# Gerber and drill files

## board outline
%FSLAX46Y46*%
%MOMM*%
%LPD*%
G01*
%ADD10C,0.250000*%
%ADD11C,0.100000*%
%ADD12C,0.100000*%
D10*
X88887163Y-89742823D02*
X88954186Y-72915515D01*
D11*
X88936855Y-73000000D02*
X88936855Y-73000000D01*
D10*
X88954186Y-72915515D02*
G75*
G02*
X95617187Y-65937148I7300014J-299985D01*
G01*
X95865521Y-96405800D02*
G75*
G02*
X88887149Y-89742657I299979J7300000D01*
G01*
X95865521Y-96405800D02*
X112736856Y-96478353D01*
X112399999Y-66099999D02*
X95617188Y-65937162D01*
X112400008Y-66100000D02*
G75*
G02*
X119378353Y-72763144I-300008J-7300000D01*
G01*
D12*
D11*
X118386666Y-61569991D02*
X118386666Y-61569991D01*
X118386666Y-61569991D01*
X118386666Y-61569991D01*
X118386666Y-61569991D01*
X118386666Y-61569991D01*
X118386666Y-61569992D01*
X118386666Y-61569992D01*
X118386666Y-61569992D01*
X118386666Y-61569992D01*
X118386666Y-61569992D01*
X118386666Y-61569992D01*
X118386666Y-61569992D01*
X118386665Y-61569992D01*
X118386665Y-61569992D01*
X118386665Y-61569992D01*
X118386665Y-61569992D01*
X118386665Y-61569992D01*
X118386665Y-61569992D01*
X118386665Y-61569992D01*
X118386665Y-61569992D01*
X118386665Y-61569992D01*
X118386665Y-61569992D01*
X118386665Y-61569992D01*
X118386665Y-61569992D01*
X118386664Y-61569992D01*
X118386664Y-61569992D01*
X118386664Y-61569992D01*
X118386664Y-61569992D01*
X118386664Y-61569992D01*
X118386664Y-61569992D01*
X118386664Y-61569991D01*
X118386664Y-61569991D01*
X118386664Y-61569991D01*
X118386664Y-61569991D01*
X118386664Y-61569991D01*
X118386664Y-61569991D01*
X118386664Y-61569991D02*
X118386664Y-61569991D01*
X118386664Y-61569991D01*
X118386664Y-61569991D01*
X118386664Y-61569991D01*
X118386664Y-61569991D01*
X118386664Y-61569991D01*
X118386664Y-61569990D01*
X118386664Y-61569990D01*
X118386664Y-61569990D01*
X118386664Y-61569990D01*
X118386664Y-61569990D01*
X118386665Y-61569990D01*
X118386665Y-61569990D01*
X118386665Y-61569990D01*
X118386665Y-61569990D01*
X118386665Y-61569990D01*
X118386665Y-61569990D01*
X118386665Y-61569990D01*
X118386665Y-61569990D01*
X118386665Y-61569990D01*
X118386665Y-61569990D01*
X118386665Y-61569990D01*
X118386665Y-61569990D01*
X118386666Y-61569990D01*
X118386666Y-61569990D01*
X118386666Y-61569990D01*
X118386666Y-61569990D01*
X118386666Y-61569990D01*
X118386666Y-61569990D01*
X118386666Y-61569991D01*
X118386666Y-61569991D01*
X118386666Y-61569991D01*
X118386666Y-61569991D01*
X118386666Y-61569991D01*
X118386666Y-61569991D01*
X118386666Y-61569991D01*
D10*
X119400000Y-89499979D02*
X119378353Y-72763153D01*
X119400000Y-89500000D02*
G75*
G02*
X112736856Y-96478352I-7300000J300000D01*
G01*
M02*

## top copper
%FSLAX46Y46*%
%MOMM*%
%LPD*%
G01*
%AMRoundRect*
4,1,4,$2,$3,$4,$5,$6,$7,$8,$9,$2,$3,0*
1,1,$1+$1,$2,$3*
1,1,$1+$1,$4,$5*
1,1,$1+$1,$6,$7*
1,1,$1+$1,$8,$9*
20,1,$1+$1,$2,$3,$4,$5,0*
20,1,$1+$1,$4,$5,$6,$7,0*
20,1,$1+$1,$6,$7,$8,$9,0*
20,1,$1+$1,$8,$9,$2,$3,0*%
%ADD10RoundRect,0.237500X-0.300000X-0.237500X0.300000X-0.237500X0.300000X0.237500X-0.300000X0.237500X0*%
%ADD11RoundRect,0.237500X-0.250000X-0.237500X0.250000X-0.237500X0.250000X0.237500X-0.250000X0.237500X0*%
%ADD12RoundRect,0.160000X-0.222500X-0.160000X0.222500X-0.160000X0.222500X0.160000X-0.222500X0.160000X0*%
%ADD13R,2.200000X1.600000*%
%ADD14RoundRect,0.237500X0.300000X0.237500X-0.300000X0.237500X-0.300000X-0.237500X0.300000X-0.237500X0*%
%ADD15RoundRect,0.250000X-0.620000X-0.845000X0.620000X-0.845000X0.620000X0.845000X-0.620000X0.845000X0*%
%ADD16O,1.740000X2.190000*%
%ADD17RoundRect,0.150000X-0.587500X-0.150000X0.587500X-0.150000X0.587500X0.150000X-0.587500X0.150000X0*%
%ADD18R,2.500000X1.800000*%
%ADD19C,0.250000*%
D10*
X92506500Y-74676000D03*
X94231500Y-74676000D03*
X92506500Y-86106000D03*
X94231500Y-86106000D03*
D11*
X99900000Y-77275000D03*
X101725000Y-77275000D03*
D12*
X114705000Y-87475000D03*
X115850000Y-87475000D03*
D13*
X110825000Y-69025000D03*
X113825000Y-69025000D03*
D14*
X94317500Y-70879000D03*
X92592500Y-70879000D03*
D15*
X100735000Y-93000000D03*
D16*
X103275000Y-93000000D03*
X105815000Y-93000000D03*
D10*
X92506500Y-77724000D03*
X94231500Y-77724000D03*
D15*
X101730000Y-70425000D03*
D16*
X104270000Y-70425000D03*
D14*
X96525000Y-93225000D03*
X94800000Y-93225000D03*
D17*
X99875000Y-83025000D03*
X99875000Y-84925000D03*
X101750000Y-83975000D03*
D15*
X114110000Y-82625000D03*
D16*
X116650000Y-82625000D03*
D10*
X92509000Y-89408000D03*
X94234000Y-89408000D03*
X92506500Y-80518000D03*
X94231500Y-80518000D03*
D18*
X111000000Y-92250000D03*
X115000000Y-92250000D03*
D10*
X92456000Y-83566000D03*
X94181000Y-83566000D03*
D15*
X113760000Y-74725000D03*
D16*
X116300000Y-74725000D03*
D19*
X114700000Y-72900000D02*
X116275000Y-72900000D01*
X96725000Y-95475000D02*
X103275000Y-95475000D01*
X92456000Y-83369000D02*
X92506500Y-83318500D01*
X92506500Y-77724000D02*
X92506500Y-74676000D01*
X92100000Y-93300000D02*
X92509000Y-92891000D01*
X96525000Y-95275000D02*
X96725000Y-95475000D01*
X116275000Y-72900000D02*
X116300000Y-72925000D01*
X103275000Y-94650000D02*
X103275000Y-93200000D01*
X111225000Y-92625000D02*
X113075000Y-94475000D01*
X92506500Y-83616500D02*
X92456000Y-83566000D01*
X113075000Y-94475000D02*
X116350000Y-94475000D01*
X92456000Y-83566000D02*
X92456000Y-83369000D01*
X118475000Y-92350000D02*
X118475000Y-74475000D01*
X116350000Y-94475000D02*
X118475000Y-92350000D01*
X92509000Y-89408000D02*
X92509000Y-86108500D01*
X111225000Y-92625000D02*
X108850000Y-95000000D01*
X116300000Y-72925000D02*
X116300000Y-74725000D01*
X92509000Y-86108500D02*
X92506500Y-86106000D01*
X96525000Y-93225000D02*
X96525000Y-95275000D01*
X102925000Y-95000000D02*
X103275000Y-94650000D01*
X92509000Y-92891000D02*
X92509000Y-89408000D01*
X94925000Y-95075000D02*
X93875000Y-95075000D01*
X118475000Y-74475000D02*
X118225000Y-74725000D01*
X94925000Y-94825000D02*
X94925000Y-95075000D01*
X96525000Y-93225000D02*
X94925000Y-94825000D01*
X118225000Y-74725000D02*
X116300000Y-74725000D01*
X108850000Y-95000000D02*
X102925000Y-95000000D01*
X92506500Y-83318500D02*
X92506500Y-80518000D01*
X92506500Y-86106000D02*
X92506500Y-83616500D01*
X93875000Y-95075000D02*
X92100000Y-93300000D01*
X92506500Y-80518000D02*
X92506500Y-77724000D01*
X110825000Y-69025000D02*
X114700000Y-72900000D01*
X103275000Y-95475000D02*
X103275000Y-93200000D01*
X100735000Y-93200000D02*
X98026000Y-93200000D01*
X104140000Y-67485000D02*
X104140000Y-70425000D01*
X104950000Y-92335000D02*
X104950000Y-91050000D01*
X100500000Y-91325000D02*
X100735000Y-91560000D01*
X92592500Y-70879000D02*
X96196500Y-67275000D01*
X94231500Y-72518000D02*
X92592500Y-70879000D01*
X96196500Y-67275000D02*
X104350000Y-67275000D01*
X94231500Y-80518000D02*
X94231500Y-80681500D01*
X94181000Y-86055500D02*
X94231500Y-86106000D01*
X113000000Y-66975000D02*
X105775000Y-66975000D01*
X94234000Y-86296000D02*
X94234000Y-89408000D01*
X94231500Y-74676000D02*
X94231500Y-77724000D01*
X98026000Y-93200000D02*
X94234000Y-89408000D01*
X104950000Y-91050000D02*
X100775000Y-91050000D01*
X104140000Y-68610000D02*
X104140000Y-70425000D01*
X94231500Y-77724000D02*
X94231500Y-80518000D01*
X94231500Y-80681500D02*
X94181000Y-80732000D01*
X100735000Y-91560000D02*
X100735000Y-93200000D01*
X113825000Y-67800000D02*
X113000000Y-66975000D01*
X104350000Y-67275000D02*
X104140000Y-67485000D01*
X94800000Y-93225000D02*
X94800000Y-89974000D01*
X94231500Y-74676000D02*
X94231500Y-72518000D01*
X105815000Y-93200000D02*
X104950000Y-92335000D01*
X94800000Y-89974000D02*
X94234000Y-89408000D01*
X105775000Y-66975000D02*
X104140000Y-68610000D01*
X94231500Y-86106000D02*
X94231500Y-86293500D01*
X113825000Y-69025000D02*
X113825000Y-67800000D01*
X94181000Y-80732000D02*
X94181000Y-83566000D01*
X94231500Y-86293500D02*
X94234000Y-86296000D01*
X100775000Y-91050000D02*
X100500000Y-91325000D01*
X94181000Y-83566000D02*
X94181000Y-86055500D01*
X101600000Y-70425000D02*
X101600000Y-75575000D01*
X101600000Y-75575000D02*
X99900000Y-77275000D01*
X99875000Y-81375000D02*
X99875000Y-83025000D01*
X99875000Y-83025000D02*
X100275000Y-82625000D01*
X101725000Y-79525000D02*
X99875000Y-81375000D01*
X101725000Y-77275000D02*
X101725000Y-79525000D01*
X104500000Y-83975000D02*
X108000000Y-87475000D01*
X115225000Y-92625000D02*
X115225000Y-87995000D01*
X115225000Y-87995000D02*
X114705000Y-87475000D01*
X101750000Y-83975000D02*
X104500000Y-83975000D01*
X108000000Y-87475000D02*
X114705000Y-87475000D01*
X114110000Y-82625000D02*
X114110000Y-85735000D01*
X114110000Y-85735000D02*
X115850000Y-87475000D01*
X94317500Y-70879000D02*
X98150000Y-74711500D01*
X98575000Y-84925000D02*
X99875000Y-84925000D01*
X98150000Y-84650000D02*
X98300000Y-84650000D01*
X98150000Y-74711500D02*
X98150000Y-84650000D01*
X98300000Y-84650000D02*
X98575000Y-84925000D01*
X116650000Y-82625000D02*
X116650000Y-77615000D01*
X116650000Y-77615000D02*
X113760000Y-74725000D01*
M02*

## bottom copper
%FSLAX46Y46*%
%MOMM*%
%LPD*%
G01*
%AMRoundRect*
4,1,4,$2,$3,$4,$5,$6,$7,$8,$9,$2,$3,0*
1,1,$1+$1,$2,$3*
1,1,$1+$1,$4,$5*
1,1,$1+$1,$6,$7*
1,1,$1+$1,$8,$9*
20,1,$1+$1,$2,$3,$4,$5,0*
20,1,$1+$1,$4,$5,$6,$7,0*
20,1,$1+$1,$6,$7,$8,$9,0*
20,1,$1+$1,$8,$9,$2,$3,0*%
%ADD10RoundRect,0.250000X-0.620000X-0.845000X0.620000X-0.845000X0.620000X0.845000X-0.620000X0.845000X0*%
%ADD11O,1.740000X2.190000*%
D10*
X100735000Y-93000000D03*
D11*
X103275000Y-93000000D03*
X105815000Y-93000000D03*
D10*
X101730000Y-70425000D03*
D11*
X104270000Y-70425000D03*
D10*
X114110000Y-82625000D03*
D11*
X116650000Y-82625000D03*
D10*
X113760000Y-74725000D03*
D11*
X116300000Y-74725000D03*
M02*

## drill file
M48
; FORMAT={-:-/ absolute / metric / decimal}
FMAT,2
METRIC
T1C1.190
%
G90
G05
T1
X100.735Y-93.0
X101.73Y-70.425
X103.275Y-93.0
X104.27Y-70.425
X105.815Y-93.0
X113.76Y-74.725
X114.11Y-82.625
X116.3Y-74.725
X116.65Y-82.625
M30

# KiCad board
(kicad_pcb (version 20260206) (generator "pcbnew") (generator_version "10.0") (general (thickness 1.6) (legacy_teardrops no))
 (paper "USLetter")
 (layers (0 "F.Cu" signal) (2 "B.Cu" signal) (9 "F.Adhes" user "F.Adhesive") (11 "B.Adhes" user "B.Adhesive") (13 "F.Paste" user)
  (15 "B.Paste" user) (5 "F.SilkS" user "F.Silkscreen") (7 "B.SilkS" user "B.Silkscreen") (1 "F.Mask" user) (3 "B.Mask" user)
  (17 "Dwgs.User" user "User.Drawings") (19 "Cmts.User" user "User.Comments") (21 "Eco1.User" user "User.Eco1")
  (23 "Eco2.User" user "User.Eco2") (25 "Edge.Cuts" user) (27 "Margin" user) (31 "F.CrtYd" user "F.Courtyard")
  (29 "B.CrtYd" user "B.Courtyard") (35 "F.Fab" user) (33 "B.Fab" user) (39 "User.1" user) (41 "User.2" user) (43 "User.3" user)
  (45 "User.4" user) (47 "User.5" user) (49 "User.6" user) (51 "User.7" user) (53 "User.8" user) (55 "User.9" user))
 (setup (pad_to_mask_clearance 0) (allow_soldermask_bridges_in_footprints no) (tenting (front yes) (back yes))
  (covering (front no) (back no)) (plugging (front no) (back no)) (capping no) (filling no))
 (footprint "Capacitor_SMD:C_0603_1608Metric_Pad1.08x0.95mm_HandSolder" (layer "F.Cu") (at 93.369 74.676)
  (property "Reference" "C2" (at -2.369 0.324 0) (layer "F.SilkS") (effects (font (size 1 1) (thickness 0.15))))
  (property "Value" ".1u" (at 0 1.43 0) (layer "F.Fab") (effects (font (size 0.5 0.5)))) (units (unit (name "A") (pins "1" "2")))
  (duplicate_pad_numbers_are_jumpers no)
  (pad "1" smd roundrect (at -0.8625 0) (size 1.075 0.95) (layers "F.Cu" "F.Mask" "F.Paste") (roundrect_rratio 0.25) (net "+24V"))
  (pad "2" smd roundrect (at 0.8625 0) (size 1.075 0.95) (layers "F.Cu" "F.Mask" "F.Paste") (roundrect_rratio 0.25) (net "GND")))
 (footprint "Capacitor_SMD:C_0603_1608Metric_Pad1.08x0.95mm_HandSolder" (layer "F.Cu") (at 93.369 86.106)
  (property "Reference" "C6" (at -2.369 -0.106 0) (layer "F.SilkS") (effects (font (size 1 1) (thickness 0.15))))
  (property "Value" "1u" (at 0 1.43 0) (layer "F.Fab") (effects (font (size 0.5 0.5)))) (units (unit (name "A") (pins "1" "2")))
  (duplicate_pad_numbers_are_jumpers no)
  (pad "1" smd roundrect (at -0.8625 0) (size 1.075 0.95) (layers "F.Cu" "F.Mask" "F.Paste") (roundrect_rratio 0.25) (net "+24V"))
  (pad "2" smd roundrect (at 0.8625 0) (size 1.075 0.95) (layers "F.Cu" "F.Mask" "F.Paste") (roundrect_rratio 0.25) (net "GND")))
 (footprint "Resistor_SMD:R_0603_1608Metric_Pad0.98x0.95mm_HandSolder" (layer "F.Cu") (at 100.8125 77.275)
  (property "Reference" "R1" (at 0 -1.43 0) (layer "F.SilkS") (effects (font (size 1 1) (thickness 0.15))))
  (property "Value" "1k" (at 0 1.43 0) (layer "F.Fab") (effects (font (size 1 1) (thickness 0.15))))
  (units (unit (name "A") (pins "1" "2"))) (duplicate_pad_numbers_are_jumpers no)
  (pad "1" smd roundrect (at -0.9125 0) (size 0.975 0.95) (layers "F.Cu" "F.Mask" "F.Paste") (roundrect_rratio 0.25) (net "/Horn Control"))
  (pad "2" smd roundrect (at 0.9125 0) (size 0.975 0.95) (layers "F.Cu" "F.Mask" "F.Paste") (roundrect_rratio 0.25) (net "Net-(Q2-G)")))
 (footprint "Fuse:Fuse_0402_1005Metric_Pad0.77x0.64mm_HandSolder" (layer "F.Cu") (at 115.2775 87.475)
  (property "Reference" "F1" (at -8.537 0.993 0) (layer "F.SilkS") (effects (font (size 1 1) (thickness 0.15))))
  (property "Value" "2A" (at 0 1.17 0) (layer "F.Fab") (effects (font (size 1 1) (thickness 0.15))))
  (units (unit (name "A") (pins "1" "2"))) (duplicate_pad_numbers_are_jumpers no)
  (pad "1" smd roundrect (at -0.5725 0) (size 0.765 0.64) (layers "F.Cu" "F.Mask" "F.Paste") (roundrect_rratio 0.25) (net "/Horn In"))
  (pad "2" smd roundrect (at 0.5725 0) (size 0.765 0.64) (layers "F.Cu" "F.Mask" "F.Paste") (roundrect_rratio 0.25) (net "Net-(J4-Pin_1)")))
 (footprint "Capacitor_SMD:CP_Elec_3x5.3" (layer "F.Cu") (at 112.325 69.025)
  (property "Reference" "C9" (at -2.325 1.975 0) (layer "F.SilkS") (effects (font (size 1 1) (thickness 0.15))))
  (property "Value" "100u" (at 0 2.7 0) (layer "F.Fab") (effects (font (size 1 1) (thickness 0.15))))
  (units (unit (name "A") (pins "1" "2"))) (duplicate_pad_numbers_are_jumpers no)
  (pad "1" smd rect (at -1.5 0) (size 2.2 1.6) (layers "F.Cu" "F.Mask" "F.Paste") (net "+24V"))
  (pad "2" smd rect (at 1.5 0) (size 2.2 1.6) (layers "F.Cu" "F.Mask" "F.Paste") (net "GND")))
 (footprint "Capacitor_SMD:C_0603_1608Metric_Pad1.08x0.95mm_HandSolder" (layer "F.Cu") (at 93.455 70.879 180)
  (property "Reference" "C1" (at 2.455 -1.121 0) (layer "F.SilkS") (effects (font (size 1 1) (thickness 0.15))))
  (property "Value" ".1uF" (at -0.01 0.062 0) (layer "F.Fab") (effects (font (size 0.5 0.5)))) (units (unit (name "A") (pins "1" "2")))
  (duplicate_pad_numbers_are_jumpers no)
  (pad "1" smd roundrect (at -0.8625 0 180) (size 1.075 0.95) (layers "F.Cu" "F.Mask" "F.Paste") (roundrect_rratio 0.25) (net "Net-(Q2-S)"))
  (pad "2" smd roundrect (at 0.8625 0 180) (size 1.075 0.95) (layers "F.Cu" "F.Mask" "F.Paste") (roundrect_rratio 0.25) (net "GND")))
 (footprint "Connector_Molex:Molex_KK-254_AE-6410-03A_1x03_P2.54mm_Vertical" (layer "F.Cu") (at 100.735 93)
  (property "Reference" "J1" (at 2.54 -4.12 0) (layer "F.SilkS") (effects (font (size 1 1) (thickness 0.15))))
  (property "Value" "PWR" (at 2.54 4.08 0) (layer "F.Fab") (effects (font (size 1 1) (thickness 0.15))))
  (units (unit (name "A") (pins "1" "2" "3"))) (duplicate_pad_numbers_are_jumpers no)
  (pad "1" thru_hole roundrect (at 0 0) (size 1.74 2.19) (drill 1.19) (layers "*.Cu" "*.Mask") (remove_unused_layers no)
   (roundrect_rratio 0.143678) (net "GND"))
  (pad "2" thru_hole oval (at 2.54 0) (size 1.74 2.19) (drill 1.19) (layers "*.Cu" "*.Mask") (remove_unused_layers no) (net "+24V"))
  (pad "3" thru_hole oval (at 5.08 0) (size 1.74 2.19) (drill 1.19) (layers "*.Cu" "*.Mask") (remove_unused_layers no) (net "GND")))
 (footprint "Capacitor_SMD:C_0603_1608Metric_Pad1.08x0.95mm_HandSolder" (layer "F.Cu") (at 93.369 77.724)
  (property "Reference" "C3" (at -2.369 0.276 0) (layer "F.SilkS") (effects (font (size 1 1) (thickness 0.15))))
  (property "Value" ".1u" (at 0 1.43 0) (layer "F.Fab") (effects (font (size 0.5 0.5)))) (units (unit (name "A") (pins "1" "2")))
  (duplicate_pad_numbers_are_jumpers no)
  (pad "1" smd roundrect (at -0.8625 0) (size 1.075 0.95) (layers "F.Cu" "F.Mask" "F.Paste") (roundrect_rratio 0.25) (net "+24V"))
  (pad "2" smd roundrect (at 0.8625 0) (size 1.075 0.95) (layers "F.Cu" "F.Mask" "F.Paste") (roundrect_rratio 0.25) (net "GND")))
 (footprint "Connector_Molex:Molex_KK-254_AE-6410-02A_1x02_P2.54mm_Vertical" (layer "F.Cu") (at 101.73 70.425)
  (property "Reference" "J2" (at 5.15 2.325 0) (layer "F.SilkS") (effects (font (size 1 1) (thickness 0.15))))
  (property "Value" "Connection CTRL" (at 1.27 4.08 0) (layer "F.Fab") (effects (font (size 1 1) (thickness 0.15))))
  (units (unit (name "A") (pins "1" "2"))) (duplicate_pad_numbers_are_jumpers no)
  (pad "1" thru_hole roundrect (at 0 0) (size 1.74 2.19) (drill 1.19) (layers "*.Cu" "*.Mask") (remove_unused_layers no)
   (roundrect_rratio 0.143678) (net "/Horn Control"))
  (pad "2" thru_hole oval (at 2.54 0) (size 1.74 2.19) (drill 1.19) (layers "*.Cu" "*.Mask") (remove_unused_layers no) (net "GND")))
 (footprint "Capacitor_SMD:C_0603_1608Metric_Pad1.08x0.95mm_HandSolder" (layer "F.Cu") (at 95.6625 93.225 180)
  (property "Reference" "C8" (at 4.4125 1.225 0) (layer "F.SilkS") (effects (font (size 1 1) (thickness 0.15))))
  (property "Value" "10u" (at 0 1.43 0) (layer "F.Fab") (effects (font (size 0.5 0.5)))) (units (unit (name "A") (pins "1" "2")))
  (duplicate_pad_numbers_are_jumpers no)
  (pad "1" smd roundrect (at -0.8625 0 180) (size 1.075 0.95) (layers "F.Cu" "F.Mask" "F.Paste") (roundrect_rratio 0.25) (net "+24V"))
  (pad "2" smd roundrect (at 0.8625 0 180) (size 1.075 0.95) (layers "F.Cu" "F.Mask" "F.Paste") (roundrect_rratio 0.25) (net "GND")))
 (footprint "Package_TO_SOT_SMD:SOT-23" (layer "F.Cu") (at 100.8125 83.975)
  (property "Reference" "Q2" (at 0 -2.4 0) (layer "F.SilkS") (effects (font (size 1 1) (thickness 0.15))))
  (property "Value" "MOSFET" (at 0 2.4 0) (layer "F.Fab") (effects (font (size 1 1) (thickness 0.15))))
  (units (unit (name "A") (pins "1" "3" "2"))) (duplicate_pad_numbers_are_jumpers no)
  (pad "1" smd roundrect (at -0.9375 -0.95) (size 1.475 0.6) (layers "F.Cu" "F.Mask" "F.Paste") (roundrect_rratio 0.25) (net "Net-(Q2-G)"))
  (pad "2" smd roundrect (at -0.9375 0.95) (size 1.475 0.6) (layers "F.Cu" "F.Mask" "F.Paste") (roundrect_rratio 0.25) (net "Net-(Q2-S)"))
  (pad "3" smd roundrect (at 0.9375 0) (size 1.475 0.6) (layers "F.Cu" "F.Mask" "F.Paste") (roundrect_rratio 0.25) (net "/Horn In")))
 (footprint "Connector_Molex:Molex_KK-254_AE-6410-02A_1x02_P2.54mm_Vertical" (layer "F.Cu") (at 114.11 82.625)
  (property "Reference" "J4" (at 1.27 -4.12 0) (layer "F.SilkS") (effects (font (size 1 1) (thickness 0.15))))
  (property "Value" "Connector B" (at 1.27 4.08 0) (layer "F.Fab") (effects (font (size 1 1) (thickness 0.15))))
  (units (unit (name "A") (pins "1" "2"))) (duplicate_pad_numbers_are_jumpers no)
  (pad "1" thru_hole roundrect (at 0 0) (size 1.74 2.19) (drill 1.19) (layers "*.Cu" "*.Mask") (remove_unused_layers no)
   (roundrect_rratio 0.143678) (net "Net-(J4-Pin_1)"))
  (pad "2" thru_hole oval (at 2.54 0) (size 1.74 2.19) (drill 1.19) (layers "*.Cu" "*.Mask") (remove_unused_layers no)
   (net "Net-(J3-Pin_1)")))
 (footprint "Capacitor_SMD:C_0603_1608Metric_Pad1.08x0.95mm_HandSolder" (layer "F.Cu") (at 93.3715 89.408)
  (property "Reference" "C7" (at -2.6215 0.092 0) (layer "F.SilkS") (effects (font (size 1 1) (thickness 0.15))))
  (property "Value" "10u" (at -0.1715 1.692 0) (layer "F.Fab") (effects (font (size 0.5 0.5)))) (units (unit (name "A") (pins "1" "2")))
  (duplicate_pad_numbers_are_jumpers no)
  (pad "1" smd roundrect (at -0.8625 0) (size 1.075 0.95) (layers "F.Cu" "F.Mask" "F.Paste") (roundrect_rratio 0.25) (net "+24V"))
  (pad "2" smd roundrect (at 0.8625 0) (size 1.075 0.95) (layers "F.Cu" "F.Mask" "F.Paste") (roundrect_rratio 0.25) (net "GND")))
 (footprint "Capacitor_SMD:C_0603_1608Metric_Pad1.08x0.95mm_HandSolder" (layer "F.Cu") (at 93.369 80.518)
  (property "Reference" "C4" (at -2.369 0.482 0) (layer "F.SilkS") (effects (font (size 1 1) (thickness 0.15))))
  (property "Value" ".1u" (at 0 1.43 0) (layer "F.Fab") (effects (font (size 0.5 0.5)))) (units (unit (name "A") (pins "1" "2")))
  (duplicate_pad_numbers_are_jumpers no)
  (pad "1" smd roundrect (at -0.8625 0) (size 1.075 0.95) (layers "F.Cu" "F.Mask" "F.Paste") (roundrect_rratio 0.25) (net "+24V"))
  (pad "2" smd roundrect (at 0.8625 0) (size 1.075 0.95) (layers "F.Cu" "F.Mask" "F.Paste") (roundrect_rratio 0.25) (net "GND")))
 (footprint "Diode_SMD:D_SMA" (layer "F.Cu") (at 113 92.25)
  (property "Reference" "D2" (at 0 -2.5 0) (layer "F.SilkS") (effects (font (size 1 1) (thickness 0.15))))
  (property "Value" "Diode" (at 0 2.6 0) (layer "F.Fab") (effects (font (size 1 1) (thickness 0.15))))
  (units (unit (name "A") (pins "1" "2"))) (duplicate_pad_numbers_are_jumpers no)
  (pad "1" smd rect (at -2 0) (size 2.5 1.8) (layers "F.Cu" "F.Mask" "F.Paste") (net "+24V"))
  (pad "2" smd rect (at 2 0) (size 2.5 1.8) (layers "F.Cu" "F.Mask" "F.Paste") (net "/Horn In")))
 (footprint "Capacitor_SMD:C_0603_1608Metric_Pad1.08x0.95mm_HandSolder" (layer "F.Cu") (at 93.3185 83.566)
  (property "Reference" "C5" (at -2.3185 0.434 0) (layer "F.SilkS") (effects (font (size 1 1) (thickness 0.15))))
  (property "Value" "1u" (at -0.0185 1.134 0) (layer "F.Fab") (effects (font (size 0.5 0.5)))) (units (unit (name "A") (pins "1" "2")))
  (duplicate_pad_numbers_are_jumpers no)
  (pad "1" smd roundrect (at -0.8625 0) (size 1.075 0.95) (layers "F.Cu" "F.Mask" "F.Paste") (roundrect_rratio 0.25) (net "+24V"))
  (pad "2" smd roundrect (at 0.8625 0) (size 1.075 0.95) (layers "F.Cu" "F.Mask" "F.Paste") (roundrect_rratio 0.25) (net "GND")))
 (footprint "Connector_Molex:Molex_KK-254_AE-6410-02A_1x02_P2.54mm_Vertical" (layer "F.Cu") (at 113.76 74.725)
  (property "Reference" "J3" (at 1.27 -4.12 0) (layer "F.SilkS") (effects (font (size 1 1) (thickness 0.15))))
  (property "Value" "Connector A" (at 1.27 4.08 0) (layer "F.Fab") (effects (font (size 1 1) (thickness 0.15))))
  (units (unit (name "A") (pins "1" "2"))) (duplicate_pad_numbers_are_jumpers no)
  (pad "1" thru_hole roundrect (at 0 0) (size 1.74 2.19) (drill 1.19) (layers "*.Cu" "*.Mask") (remove_unused_layers no)
   (roundrect_rratio 0.143678) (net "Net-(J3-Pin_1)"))
  (pad "2" thru_hole oval (at 2.54 0) (size 1.74 2.19) (drill 1.19) (layers "*.Cu" "*.Mask") (remove_unused_layers no) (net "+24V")))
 (gr_line (start 88.887163 89.742823) (end 88.954186 72.915515) (stroke (width 0.25) (type solid)) (layer "Edge.Cuts"))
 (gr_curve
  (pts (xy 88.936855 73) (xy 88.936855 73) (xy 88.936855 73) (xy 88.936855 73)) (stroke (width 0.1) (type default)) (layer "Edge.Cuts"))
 (gr_arc (start 88.954186 72.915515) (mid 90.969936 68.170046) (end 95.617188 65.937162) (stroke (width 0.25) (type solid))
  (layer "Edge.Cuts"))
 (gr_arc (start 95.865521 96.4058) (mid 91.120002 94.390002) (end 88.887162 89.742656) (stroke (width 0.25) (type solid))
  (layer "Edge.Cuts"))
 (gr_line (start 95.865521 96.4058) (end 112.736856 96.478353) (stroke (width 0.25) (type solid)) (layer "Edge.Cuts"))
 (gr_line (start 112.399999 66.099999) (end 95.617188 65.937162) (stroke (width 0.25) (type solid)) (layer "Edge.Cuts"))
 (gr_arc (start 112.400008 66.1) (mid 117.145519 68.115802) (end 119.378353 72.763144) (stroke (width 0.25) (type solid))
  (layer "Edge.Cuts"))
 (gr_arc (start 118.386665 61.569991) (mid 118.386665 61.569991) (end 118.386665 61.569991) (stroke (width 0.1) (type default))
  (layer "Edge.Cuts"))
 (gr_line (start 119.4 89.499979) (end 119.378353 72.763153) (stroke (width 0.25) (type solid)) (layer "Edge.Cuts"))
 (gr_arc (start 119.4 89.5) (mid 117.3842 94.245516) (end 112.736856 96.478353) (stroke (width 0.25) (type solid)) (layer "Edge.Cuts"))
 (segment (start 114.7 72.9) (end 116.275 72.9) (width 0.25) (layer "F.Cu") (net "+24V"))
 (segment (start 96.725 95.475) (end 103.275 95.475) (width 0.25) (layer "F.Cu") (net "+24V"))
 (segment (start 92.456 83.369) (end 92.5065 83.3185) (width 0.25) (layer "F.Cu") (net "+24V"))
 (segment (start 92.5065 77.724) (end 92.5065 74.676) (width 0.25) (layer "F.Cu") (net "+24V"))
 (segment (start 92.1 93.3) (end 92.509 92.891) (width 0.25) (layer "F.Cu") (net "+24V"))
 (segment (start 96.525 95.275) (end 96.725 95.475) (width 0.25) (layer "F.Cu") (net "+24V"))
 (segment (start 116.275 72.9) (end 116.3 72.925) (width 0.25) (layer "F.Cu") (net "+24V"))
 (segment (start 103.275 94.65) (end 103.275 93.2) (width 0.25) (layer "F.Cu") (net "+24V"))
 (segment (start 111.225 92.625) (end 113.075 94.475) (width 0.25) (layer "F.Cu") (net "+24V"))
 (segment (start 92.5065 83.6165) (end 92.456 83.566) (width 0.25) (layer "F.Cu") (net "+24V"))
 (segment (start 113.075 94.475) (end 116.35 94.475) (width 0.25) (layer "F.Cu") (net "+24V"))
 (segment (start 92.456 83.566) (end 92.456 83.369) (width 0.25) (layer "F.Cu") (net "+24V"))
 (segment (start 118.475 92.35) (end 118.475 74.475) (width 0.25) (layer "F.Cu") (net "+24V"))
 (segment (start 116.35 94.475) (end 118.475 92.35) (width 0.25) (layer "F.Cu") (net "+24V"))
 (segment (start 92.509 89.408) (end 92.509 86.1085) (width 0.25) (layer "F.Cu") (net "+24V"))
 (segment (start 111.225 92.625) (end 108.85 95) (width 0.25) (layer "F.Cu") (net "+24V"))
 (segment (start 116.3 72.925) (end 116.3 74.725) (width 0.25) (layer "F.Cu") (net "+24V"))
 (segment (start 92.509 86.1085) (end 92.5065 86.106) (width 0.25) (layer "F.Cu") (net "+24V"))
 (segment (start 96.525 93.225) (end 96.525 95.275) (width 0.25) (layer "F.Cu") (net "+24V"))
 (segment (start 102.925 95) (end 103.275 94.65) (width 0.25) (layer "F.Cu") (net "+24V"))
 (segment (start 92.509 92.891) (end 92.509 89.408) (width 0.25) (layer "F.Cu") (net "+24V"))
 (segment (start 94.925 95.075) (end 93.875 95.075) (width 0.25) (layer "F.Cu") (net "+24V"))
 (segment (start 118.475 74.475) (end 118.225 74.725) (width 0.25) (layer "F.Cu") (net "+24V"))
 (segment (start 94.925 94.825) (end 94.925 95.075) (width 0.25) (layer "F.Cu") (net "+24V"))
 (segment (start 96.525 93.225) (end 94.925 94.825) (width 0.25) (layer "F.Cu") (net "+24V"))
 (segment (start 118.225 74.725) (end 116.3 74.725) (width 0.25) (layer "F.Cu") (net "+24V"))
 (segment (start 108.85 95) (end 102.925 95) (width 0.25) (layer "F.Cu") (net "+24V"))
 (segment (start 92.5065 83.3185) (end 92.5065 80.518) (width 0.25) (layer "F.Cu") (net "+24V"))
 (segment (start 92.5065 86.106) (end 92.5065 83.6165) (width 0.25) (layer "F.Cu") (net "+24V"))
 (segment (start 93.875 95.075) (end 92.1 93.3) (width 0.25) (layer "F.Cu") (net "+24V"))
 (segment (start 92.5065 80.518) (end 92.5065 77.724) (width 0.25) (layer "F.Cu") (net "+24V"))
 (segment (start 110.825 69.025) (end 114.7 72.9) (width 0.25) (layer "F.Cu") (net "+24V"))
 (segment (start 103.275 95.475) (end 103.275 93.2) (width 0.25) (layer "F.Cu") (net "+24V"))
 (segment (start 100.735 93.2) (end 98.026 93.2) (width 0.25) (layer "F.Cu") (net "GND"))
 (segment (start 104.14 67.485) (end 104.14 70.425) (width 0.25) (layer "F.Cu") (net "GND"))
 (segment (start 104.95 92.335) (end 104.95 91.05) (width 0.25) (layer "F.Cu") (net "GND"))
 (segment (start 100.5 91.325) (end 100.735 91.56) (width 0.25) (layer "F.Cu") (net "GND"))
 (segment (start 92.5925 70.879) (end 96.1965 67.275) (width 0.25) (layer "F.Cu") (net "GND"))
 (segment (start 94.2315 72.518) (end 92.5925 70.879) (width 0.25) (layer "F.Cu") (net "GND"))
 (segment (start 96.1965 67.275) (end 104.35 67.275) (width 0.25) (layer "F.Cu") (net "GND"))
 (segment (start 94.2315 80.518) (end 94.2315 80.6815) (width 0.25) (layer "F.Cu") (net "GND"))
 (segment (start 94.181 86.0555) (end 94.2315 86.106) (width 0.25) (layer "F.Cu") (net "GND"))
 (segment (start 113 66.975) (end 105.775 66.975) (width 0.25) (layer "F.Cu") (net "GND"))
 (segment (start 94.234 86.296) (end 94.234 89.408) (width 0.25) (layer "F.Cu") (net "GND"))
 (segment (start 94.2315 74.676) (end 94.2315 77.724) (width 0.25) (layer "F.Cu") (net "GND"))
 (segment (start 98.026 93.2) (end 94.234 89.408) (width 0.25) (layer "F.Cu") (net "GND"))
 (segment (start 104.95 91.05) (end 100.775 91.05) (width 0.25) (layer "F.Cu") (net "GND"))
 (segment (start 104.14 68.61) (end 104.14 70.425) (width 0.25) (layer "F.Cu") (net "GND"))
 (segment (start 94.2315 77.724) (end 94.2315 80.518) (width 0.25) (layer "F.Cu") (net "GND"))
 (segment (start 94.2315 80.6815) (end 94.181 80.732) (width 0.25) (layer "F.Cu") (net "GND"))
 (segment (start 100.735 91.56) (end 100.735 93.2) (width 0.25) (layer "F.Cu") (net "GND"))
 (segment (start 113.825 67.8) (end 113 66.975) (width 0.25) (layer "F.Cu") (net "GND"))
 (segment (start 104.35 67.275) (end 104.14 67.485) (width 0.25) (layer "F.Cu") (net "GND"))
 (segment (start 94.8 93.225) (end 94.8 89.974) (width 0.25) (layer "F.Cu") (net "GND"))
 (segment (start 94.2315 74.676) (end 94.2315 72.518) (width 0.25) (layer "F.Cu") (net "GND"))
 (segment (start 105.815 93.2) (end 104.95 92.335) (width 0.25) (layer "F.Cu") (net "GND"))
 (segment (start 94.8 89.974) (end 94.234 89.408) (width 0.25) (layer "F.Cu") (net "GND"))
 (segment (start 105.775 66.975) (end 104.14 68.61) (width 0.25) (layer "F.Cu") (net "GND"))
 (segment (start 94.2315 86.106) (end 94.2315 86.2935) (width 0.25) (layer "F.Cu") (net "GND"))
 (segment (start 113.825 69.025) (end 113.825 67.8) (width 0.25) (layer "F.Cu") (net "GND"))
 (segment (start 94.181 80.732) (end 94.181 83.566) (width 0.25) (layer "F.Cu") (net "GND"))
 (segment (start 94.2315 86.2935) (end 94.234 86.296) (width 0.25) (layer "F.Cu") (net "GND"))
 (segment (start 100.775 91.05) (end 100.5 91.325) (width 0.25) (layer "F.Cu") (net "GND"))
 (segment (start 94.181 83.566) (end 94.181 86.0555) (width 0.25) (layer "F.Cu") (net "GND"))
 (segment (start 101.6 70.425) (end 101.6 75.575) (width 0.25) (layer "F.Cu") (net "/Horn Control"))
 (segment (start 101.6 75.575) (end 99.9 77.275) (width 0.25) (layer "F.Cu") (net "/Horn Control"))
 (segment (start 99.875 81.375) (end 99.875 83.025) (width 0.25) (layer "F.Cu") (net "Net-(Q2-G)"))
 (segment (start 99.875 83.025) (end 100.275 82.625) (width 0.25) (layer "F.Cu") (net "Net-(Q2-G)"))
 (segment (start 101.725 79.525) (end 99.875 81.375) (width 0.25) (layer "F.Cu") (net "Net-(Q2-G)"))
 (segment (start 101.725 77.275) (end 101.725 79.525) (width 0.25) (layer "F.Cu") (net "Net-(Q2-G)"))
 (segment (start 104.5 83.975) (end 108 87.475) (width 0.25) (layer "F.Cu") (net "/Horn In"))
 (segment (start 115.225 92.625) (end 115.225 87.995) (width 0.25) (layer "F.Cu") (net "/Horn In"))
 (segment (start 115.225 87.995) (end 114.705 87.475) (width 0.25) (layer "F.Cu") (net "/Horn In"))
 (segment (start 101.75 83.975) (end 104.5 83.975) (width 0.25) (layer "F.Cu") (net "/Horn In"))
 (segment (start 108 87.475) (end 114.705 87.475) (width 0.25) (layer "F.Cu") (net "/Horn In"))
 (segment (start 114.11 82.625) (end 114.11 85.735) (width 0.25) (layer "F.Cu") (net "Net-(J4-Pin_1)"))
 (segment (start 114.11 85.735) (end 115.85 87.475) (width 0.25) (layer "F.Cu") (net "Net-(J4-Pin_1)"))
 (segment (start 94.3175 70.879) (end 98.15 74.7115) (width 0.25) (layer "F.Cu") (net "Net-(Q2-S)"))
 (segment (start 98.575 84.925) (end 99.875 84.925) (width 0.25) (layer "F.Cu") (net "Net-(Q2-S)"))
 (segment (start 98.15 84.65) (end 98.3 84.65) (width 0.25) (layer "F.Cu") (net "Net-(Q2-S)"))
 (segment (start 98.15 74.7115) (end 98.15 84.65) (width 0.25) (layer "F.Cu") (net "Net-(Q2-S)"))
 (segment (start 98.3 84.65) (end 98.575 84.925) (width 0.25) (layer "F.Cu") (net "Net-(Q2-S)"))
 (segment (start 116.65 82.625) (end 116.65 77.615) (width 0.25) (layer "F.Cu") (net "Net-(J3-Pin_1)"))
 (segment (start 116.65 77.615) (end 113.76 74.725) (width 0.25) (layer "F.Cu") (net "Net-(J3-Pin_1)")))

